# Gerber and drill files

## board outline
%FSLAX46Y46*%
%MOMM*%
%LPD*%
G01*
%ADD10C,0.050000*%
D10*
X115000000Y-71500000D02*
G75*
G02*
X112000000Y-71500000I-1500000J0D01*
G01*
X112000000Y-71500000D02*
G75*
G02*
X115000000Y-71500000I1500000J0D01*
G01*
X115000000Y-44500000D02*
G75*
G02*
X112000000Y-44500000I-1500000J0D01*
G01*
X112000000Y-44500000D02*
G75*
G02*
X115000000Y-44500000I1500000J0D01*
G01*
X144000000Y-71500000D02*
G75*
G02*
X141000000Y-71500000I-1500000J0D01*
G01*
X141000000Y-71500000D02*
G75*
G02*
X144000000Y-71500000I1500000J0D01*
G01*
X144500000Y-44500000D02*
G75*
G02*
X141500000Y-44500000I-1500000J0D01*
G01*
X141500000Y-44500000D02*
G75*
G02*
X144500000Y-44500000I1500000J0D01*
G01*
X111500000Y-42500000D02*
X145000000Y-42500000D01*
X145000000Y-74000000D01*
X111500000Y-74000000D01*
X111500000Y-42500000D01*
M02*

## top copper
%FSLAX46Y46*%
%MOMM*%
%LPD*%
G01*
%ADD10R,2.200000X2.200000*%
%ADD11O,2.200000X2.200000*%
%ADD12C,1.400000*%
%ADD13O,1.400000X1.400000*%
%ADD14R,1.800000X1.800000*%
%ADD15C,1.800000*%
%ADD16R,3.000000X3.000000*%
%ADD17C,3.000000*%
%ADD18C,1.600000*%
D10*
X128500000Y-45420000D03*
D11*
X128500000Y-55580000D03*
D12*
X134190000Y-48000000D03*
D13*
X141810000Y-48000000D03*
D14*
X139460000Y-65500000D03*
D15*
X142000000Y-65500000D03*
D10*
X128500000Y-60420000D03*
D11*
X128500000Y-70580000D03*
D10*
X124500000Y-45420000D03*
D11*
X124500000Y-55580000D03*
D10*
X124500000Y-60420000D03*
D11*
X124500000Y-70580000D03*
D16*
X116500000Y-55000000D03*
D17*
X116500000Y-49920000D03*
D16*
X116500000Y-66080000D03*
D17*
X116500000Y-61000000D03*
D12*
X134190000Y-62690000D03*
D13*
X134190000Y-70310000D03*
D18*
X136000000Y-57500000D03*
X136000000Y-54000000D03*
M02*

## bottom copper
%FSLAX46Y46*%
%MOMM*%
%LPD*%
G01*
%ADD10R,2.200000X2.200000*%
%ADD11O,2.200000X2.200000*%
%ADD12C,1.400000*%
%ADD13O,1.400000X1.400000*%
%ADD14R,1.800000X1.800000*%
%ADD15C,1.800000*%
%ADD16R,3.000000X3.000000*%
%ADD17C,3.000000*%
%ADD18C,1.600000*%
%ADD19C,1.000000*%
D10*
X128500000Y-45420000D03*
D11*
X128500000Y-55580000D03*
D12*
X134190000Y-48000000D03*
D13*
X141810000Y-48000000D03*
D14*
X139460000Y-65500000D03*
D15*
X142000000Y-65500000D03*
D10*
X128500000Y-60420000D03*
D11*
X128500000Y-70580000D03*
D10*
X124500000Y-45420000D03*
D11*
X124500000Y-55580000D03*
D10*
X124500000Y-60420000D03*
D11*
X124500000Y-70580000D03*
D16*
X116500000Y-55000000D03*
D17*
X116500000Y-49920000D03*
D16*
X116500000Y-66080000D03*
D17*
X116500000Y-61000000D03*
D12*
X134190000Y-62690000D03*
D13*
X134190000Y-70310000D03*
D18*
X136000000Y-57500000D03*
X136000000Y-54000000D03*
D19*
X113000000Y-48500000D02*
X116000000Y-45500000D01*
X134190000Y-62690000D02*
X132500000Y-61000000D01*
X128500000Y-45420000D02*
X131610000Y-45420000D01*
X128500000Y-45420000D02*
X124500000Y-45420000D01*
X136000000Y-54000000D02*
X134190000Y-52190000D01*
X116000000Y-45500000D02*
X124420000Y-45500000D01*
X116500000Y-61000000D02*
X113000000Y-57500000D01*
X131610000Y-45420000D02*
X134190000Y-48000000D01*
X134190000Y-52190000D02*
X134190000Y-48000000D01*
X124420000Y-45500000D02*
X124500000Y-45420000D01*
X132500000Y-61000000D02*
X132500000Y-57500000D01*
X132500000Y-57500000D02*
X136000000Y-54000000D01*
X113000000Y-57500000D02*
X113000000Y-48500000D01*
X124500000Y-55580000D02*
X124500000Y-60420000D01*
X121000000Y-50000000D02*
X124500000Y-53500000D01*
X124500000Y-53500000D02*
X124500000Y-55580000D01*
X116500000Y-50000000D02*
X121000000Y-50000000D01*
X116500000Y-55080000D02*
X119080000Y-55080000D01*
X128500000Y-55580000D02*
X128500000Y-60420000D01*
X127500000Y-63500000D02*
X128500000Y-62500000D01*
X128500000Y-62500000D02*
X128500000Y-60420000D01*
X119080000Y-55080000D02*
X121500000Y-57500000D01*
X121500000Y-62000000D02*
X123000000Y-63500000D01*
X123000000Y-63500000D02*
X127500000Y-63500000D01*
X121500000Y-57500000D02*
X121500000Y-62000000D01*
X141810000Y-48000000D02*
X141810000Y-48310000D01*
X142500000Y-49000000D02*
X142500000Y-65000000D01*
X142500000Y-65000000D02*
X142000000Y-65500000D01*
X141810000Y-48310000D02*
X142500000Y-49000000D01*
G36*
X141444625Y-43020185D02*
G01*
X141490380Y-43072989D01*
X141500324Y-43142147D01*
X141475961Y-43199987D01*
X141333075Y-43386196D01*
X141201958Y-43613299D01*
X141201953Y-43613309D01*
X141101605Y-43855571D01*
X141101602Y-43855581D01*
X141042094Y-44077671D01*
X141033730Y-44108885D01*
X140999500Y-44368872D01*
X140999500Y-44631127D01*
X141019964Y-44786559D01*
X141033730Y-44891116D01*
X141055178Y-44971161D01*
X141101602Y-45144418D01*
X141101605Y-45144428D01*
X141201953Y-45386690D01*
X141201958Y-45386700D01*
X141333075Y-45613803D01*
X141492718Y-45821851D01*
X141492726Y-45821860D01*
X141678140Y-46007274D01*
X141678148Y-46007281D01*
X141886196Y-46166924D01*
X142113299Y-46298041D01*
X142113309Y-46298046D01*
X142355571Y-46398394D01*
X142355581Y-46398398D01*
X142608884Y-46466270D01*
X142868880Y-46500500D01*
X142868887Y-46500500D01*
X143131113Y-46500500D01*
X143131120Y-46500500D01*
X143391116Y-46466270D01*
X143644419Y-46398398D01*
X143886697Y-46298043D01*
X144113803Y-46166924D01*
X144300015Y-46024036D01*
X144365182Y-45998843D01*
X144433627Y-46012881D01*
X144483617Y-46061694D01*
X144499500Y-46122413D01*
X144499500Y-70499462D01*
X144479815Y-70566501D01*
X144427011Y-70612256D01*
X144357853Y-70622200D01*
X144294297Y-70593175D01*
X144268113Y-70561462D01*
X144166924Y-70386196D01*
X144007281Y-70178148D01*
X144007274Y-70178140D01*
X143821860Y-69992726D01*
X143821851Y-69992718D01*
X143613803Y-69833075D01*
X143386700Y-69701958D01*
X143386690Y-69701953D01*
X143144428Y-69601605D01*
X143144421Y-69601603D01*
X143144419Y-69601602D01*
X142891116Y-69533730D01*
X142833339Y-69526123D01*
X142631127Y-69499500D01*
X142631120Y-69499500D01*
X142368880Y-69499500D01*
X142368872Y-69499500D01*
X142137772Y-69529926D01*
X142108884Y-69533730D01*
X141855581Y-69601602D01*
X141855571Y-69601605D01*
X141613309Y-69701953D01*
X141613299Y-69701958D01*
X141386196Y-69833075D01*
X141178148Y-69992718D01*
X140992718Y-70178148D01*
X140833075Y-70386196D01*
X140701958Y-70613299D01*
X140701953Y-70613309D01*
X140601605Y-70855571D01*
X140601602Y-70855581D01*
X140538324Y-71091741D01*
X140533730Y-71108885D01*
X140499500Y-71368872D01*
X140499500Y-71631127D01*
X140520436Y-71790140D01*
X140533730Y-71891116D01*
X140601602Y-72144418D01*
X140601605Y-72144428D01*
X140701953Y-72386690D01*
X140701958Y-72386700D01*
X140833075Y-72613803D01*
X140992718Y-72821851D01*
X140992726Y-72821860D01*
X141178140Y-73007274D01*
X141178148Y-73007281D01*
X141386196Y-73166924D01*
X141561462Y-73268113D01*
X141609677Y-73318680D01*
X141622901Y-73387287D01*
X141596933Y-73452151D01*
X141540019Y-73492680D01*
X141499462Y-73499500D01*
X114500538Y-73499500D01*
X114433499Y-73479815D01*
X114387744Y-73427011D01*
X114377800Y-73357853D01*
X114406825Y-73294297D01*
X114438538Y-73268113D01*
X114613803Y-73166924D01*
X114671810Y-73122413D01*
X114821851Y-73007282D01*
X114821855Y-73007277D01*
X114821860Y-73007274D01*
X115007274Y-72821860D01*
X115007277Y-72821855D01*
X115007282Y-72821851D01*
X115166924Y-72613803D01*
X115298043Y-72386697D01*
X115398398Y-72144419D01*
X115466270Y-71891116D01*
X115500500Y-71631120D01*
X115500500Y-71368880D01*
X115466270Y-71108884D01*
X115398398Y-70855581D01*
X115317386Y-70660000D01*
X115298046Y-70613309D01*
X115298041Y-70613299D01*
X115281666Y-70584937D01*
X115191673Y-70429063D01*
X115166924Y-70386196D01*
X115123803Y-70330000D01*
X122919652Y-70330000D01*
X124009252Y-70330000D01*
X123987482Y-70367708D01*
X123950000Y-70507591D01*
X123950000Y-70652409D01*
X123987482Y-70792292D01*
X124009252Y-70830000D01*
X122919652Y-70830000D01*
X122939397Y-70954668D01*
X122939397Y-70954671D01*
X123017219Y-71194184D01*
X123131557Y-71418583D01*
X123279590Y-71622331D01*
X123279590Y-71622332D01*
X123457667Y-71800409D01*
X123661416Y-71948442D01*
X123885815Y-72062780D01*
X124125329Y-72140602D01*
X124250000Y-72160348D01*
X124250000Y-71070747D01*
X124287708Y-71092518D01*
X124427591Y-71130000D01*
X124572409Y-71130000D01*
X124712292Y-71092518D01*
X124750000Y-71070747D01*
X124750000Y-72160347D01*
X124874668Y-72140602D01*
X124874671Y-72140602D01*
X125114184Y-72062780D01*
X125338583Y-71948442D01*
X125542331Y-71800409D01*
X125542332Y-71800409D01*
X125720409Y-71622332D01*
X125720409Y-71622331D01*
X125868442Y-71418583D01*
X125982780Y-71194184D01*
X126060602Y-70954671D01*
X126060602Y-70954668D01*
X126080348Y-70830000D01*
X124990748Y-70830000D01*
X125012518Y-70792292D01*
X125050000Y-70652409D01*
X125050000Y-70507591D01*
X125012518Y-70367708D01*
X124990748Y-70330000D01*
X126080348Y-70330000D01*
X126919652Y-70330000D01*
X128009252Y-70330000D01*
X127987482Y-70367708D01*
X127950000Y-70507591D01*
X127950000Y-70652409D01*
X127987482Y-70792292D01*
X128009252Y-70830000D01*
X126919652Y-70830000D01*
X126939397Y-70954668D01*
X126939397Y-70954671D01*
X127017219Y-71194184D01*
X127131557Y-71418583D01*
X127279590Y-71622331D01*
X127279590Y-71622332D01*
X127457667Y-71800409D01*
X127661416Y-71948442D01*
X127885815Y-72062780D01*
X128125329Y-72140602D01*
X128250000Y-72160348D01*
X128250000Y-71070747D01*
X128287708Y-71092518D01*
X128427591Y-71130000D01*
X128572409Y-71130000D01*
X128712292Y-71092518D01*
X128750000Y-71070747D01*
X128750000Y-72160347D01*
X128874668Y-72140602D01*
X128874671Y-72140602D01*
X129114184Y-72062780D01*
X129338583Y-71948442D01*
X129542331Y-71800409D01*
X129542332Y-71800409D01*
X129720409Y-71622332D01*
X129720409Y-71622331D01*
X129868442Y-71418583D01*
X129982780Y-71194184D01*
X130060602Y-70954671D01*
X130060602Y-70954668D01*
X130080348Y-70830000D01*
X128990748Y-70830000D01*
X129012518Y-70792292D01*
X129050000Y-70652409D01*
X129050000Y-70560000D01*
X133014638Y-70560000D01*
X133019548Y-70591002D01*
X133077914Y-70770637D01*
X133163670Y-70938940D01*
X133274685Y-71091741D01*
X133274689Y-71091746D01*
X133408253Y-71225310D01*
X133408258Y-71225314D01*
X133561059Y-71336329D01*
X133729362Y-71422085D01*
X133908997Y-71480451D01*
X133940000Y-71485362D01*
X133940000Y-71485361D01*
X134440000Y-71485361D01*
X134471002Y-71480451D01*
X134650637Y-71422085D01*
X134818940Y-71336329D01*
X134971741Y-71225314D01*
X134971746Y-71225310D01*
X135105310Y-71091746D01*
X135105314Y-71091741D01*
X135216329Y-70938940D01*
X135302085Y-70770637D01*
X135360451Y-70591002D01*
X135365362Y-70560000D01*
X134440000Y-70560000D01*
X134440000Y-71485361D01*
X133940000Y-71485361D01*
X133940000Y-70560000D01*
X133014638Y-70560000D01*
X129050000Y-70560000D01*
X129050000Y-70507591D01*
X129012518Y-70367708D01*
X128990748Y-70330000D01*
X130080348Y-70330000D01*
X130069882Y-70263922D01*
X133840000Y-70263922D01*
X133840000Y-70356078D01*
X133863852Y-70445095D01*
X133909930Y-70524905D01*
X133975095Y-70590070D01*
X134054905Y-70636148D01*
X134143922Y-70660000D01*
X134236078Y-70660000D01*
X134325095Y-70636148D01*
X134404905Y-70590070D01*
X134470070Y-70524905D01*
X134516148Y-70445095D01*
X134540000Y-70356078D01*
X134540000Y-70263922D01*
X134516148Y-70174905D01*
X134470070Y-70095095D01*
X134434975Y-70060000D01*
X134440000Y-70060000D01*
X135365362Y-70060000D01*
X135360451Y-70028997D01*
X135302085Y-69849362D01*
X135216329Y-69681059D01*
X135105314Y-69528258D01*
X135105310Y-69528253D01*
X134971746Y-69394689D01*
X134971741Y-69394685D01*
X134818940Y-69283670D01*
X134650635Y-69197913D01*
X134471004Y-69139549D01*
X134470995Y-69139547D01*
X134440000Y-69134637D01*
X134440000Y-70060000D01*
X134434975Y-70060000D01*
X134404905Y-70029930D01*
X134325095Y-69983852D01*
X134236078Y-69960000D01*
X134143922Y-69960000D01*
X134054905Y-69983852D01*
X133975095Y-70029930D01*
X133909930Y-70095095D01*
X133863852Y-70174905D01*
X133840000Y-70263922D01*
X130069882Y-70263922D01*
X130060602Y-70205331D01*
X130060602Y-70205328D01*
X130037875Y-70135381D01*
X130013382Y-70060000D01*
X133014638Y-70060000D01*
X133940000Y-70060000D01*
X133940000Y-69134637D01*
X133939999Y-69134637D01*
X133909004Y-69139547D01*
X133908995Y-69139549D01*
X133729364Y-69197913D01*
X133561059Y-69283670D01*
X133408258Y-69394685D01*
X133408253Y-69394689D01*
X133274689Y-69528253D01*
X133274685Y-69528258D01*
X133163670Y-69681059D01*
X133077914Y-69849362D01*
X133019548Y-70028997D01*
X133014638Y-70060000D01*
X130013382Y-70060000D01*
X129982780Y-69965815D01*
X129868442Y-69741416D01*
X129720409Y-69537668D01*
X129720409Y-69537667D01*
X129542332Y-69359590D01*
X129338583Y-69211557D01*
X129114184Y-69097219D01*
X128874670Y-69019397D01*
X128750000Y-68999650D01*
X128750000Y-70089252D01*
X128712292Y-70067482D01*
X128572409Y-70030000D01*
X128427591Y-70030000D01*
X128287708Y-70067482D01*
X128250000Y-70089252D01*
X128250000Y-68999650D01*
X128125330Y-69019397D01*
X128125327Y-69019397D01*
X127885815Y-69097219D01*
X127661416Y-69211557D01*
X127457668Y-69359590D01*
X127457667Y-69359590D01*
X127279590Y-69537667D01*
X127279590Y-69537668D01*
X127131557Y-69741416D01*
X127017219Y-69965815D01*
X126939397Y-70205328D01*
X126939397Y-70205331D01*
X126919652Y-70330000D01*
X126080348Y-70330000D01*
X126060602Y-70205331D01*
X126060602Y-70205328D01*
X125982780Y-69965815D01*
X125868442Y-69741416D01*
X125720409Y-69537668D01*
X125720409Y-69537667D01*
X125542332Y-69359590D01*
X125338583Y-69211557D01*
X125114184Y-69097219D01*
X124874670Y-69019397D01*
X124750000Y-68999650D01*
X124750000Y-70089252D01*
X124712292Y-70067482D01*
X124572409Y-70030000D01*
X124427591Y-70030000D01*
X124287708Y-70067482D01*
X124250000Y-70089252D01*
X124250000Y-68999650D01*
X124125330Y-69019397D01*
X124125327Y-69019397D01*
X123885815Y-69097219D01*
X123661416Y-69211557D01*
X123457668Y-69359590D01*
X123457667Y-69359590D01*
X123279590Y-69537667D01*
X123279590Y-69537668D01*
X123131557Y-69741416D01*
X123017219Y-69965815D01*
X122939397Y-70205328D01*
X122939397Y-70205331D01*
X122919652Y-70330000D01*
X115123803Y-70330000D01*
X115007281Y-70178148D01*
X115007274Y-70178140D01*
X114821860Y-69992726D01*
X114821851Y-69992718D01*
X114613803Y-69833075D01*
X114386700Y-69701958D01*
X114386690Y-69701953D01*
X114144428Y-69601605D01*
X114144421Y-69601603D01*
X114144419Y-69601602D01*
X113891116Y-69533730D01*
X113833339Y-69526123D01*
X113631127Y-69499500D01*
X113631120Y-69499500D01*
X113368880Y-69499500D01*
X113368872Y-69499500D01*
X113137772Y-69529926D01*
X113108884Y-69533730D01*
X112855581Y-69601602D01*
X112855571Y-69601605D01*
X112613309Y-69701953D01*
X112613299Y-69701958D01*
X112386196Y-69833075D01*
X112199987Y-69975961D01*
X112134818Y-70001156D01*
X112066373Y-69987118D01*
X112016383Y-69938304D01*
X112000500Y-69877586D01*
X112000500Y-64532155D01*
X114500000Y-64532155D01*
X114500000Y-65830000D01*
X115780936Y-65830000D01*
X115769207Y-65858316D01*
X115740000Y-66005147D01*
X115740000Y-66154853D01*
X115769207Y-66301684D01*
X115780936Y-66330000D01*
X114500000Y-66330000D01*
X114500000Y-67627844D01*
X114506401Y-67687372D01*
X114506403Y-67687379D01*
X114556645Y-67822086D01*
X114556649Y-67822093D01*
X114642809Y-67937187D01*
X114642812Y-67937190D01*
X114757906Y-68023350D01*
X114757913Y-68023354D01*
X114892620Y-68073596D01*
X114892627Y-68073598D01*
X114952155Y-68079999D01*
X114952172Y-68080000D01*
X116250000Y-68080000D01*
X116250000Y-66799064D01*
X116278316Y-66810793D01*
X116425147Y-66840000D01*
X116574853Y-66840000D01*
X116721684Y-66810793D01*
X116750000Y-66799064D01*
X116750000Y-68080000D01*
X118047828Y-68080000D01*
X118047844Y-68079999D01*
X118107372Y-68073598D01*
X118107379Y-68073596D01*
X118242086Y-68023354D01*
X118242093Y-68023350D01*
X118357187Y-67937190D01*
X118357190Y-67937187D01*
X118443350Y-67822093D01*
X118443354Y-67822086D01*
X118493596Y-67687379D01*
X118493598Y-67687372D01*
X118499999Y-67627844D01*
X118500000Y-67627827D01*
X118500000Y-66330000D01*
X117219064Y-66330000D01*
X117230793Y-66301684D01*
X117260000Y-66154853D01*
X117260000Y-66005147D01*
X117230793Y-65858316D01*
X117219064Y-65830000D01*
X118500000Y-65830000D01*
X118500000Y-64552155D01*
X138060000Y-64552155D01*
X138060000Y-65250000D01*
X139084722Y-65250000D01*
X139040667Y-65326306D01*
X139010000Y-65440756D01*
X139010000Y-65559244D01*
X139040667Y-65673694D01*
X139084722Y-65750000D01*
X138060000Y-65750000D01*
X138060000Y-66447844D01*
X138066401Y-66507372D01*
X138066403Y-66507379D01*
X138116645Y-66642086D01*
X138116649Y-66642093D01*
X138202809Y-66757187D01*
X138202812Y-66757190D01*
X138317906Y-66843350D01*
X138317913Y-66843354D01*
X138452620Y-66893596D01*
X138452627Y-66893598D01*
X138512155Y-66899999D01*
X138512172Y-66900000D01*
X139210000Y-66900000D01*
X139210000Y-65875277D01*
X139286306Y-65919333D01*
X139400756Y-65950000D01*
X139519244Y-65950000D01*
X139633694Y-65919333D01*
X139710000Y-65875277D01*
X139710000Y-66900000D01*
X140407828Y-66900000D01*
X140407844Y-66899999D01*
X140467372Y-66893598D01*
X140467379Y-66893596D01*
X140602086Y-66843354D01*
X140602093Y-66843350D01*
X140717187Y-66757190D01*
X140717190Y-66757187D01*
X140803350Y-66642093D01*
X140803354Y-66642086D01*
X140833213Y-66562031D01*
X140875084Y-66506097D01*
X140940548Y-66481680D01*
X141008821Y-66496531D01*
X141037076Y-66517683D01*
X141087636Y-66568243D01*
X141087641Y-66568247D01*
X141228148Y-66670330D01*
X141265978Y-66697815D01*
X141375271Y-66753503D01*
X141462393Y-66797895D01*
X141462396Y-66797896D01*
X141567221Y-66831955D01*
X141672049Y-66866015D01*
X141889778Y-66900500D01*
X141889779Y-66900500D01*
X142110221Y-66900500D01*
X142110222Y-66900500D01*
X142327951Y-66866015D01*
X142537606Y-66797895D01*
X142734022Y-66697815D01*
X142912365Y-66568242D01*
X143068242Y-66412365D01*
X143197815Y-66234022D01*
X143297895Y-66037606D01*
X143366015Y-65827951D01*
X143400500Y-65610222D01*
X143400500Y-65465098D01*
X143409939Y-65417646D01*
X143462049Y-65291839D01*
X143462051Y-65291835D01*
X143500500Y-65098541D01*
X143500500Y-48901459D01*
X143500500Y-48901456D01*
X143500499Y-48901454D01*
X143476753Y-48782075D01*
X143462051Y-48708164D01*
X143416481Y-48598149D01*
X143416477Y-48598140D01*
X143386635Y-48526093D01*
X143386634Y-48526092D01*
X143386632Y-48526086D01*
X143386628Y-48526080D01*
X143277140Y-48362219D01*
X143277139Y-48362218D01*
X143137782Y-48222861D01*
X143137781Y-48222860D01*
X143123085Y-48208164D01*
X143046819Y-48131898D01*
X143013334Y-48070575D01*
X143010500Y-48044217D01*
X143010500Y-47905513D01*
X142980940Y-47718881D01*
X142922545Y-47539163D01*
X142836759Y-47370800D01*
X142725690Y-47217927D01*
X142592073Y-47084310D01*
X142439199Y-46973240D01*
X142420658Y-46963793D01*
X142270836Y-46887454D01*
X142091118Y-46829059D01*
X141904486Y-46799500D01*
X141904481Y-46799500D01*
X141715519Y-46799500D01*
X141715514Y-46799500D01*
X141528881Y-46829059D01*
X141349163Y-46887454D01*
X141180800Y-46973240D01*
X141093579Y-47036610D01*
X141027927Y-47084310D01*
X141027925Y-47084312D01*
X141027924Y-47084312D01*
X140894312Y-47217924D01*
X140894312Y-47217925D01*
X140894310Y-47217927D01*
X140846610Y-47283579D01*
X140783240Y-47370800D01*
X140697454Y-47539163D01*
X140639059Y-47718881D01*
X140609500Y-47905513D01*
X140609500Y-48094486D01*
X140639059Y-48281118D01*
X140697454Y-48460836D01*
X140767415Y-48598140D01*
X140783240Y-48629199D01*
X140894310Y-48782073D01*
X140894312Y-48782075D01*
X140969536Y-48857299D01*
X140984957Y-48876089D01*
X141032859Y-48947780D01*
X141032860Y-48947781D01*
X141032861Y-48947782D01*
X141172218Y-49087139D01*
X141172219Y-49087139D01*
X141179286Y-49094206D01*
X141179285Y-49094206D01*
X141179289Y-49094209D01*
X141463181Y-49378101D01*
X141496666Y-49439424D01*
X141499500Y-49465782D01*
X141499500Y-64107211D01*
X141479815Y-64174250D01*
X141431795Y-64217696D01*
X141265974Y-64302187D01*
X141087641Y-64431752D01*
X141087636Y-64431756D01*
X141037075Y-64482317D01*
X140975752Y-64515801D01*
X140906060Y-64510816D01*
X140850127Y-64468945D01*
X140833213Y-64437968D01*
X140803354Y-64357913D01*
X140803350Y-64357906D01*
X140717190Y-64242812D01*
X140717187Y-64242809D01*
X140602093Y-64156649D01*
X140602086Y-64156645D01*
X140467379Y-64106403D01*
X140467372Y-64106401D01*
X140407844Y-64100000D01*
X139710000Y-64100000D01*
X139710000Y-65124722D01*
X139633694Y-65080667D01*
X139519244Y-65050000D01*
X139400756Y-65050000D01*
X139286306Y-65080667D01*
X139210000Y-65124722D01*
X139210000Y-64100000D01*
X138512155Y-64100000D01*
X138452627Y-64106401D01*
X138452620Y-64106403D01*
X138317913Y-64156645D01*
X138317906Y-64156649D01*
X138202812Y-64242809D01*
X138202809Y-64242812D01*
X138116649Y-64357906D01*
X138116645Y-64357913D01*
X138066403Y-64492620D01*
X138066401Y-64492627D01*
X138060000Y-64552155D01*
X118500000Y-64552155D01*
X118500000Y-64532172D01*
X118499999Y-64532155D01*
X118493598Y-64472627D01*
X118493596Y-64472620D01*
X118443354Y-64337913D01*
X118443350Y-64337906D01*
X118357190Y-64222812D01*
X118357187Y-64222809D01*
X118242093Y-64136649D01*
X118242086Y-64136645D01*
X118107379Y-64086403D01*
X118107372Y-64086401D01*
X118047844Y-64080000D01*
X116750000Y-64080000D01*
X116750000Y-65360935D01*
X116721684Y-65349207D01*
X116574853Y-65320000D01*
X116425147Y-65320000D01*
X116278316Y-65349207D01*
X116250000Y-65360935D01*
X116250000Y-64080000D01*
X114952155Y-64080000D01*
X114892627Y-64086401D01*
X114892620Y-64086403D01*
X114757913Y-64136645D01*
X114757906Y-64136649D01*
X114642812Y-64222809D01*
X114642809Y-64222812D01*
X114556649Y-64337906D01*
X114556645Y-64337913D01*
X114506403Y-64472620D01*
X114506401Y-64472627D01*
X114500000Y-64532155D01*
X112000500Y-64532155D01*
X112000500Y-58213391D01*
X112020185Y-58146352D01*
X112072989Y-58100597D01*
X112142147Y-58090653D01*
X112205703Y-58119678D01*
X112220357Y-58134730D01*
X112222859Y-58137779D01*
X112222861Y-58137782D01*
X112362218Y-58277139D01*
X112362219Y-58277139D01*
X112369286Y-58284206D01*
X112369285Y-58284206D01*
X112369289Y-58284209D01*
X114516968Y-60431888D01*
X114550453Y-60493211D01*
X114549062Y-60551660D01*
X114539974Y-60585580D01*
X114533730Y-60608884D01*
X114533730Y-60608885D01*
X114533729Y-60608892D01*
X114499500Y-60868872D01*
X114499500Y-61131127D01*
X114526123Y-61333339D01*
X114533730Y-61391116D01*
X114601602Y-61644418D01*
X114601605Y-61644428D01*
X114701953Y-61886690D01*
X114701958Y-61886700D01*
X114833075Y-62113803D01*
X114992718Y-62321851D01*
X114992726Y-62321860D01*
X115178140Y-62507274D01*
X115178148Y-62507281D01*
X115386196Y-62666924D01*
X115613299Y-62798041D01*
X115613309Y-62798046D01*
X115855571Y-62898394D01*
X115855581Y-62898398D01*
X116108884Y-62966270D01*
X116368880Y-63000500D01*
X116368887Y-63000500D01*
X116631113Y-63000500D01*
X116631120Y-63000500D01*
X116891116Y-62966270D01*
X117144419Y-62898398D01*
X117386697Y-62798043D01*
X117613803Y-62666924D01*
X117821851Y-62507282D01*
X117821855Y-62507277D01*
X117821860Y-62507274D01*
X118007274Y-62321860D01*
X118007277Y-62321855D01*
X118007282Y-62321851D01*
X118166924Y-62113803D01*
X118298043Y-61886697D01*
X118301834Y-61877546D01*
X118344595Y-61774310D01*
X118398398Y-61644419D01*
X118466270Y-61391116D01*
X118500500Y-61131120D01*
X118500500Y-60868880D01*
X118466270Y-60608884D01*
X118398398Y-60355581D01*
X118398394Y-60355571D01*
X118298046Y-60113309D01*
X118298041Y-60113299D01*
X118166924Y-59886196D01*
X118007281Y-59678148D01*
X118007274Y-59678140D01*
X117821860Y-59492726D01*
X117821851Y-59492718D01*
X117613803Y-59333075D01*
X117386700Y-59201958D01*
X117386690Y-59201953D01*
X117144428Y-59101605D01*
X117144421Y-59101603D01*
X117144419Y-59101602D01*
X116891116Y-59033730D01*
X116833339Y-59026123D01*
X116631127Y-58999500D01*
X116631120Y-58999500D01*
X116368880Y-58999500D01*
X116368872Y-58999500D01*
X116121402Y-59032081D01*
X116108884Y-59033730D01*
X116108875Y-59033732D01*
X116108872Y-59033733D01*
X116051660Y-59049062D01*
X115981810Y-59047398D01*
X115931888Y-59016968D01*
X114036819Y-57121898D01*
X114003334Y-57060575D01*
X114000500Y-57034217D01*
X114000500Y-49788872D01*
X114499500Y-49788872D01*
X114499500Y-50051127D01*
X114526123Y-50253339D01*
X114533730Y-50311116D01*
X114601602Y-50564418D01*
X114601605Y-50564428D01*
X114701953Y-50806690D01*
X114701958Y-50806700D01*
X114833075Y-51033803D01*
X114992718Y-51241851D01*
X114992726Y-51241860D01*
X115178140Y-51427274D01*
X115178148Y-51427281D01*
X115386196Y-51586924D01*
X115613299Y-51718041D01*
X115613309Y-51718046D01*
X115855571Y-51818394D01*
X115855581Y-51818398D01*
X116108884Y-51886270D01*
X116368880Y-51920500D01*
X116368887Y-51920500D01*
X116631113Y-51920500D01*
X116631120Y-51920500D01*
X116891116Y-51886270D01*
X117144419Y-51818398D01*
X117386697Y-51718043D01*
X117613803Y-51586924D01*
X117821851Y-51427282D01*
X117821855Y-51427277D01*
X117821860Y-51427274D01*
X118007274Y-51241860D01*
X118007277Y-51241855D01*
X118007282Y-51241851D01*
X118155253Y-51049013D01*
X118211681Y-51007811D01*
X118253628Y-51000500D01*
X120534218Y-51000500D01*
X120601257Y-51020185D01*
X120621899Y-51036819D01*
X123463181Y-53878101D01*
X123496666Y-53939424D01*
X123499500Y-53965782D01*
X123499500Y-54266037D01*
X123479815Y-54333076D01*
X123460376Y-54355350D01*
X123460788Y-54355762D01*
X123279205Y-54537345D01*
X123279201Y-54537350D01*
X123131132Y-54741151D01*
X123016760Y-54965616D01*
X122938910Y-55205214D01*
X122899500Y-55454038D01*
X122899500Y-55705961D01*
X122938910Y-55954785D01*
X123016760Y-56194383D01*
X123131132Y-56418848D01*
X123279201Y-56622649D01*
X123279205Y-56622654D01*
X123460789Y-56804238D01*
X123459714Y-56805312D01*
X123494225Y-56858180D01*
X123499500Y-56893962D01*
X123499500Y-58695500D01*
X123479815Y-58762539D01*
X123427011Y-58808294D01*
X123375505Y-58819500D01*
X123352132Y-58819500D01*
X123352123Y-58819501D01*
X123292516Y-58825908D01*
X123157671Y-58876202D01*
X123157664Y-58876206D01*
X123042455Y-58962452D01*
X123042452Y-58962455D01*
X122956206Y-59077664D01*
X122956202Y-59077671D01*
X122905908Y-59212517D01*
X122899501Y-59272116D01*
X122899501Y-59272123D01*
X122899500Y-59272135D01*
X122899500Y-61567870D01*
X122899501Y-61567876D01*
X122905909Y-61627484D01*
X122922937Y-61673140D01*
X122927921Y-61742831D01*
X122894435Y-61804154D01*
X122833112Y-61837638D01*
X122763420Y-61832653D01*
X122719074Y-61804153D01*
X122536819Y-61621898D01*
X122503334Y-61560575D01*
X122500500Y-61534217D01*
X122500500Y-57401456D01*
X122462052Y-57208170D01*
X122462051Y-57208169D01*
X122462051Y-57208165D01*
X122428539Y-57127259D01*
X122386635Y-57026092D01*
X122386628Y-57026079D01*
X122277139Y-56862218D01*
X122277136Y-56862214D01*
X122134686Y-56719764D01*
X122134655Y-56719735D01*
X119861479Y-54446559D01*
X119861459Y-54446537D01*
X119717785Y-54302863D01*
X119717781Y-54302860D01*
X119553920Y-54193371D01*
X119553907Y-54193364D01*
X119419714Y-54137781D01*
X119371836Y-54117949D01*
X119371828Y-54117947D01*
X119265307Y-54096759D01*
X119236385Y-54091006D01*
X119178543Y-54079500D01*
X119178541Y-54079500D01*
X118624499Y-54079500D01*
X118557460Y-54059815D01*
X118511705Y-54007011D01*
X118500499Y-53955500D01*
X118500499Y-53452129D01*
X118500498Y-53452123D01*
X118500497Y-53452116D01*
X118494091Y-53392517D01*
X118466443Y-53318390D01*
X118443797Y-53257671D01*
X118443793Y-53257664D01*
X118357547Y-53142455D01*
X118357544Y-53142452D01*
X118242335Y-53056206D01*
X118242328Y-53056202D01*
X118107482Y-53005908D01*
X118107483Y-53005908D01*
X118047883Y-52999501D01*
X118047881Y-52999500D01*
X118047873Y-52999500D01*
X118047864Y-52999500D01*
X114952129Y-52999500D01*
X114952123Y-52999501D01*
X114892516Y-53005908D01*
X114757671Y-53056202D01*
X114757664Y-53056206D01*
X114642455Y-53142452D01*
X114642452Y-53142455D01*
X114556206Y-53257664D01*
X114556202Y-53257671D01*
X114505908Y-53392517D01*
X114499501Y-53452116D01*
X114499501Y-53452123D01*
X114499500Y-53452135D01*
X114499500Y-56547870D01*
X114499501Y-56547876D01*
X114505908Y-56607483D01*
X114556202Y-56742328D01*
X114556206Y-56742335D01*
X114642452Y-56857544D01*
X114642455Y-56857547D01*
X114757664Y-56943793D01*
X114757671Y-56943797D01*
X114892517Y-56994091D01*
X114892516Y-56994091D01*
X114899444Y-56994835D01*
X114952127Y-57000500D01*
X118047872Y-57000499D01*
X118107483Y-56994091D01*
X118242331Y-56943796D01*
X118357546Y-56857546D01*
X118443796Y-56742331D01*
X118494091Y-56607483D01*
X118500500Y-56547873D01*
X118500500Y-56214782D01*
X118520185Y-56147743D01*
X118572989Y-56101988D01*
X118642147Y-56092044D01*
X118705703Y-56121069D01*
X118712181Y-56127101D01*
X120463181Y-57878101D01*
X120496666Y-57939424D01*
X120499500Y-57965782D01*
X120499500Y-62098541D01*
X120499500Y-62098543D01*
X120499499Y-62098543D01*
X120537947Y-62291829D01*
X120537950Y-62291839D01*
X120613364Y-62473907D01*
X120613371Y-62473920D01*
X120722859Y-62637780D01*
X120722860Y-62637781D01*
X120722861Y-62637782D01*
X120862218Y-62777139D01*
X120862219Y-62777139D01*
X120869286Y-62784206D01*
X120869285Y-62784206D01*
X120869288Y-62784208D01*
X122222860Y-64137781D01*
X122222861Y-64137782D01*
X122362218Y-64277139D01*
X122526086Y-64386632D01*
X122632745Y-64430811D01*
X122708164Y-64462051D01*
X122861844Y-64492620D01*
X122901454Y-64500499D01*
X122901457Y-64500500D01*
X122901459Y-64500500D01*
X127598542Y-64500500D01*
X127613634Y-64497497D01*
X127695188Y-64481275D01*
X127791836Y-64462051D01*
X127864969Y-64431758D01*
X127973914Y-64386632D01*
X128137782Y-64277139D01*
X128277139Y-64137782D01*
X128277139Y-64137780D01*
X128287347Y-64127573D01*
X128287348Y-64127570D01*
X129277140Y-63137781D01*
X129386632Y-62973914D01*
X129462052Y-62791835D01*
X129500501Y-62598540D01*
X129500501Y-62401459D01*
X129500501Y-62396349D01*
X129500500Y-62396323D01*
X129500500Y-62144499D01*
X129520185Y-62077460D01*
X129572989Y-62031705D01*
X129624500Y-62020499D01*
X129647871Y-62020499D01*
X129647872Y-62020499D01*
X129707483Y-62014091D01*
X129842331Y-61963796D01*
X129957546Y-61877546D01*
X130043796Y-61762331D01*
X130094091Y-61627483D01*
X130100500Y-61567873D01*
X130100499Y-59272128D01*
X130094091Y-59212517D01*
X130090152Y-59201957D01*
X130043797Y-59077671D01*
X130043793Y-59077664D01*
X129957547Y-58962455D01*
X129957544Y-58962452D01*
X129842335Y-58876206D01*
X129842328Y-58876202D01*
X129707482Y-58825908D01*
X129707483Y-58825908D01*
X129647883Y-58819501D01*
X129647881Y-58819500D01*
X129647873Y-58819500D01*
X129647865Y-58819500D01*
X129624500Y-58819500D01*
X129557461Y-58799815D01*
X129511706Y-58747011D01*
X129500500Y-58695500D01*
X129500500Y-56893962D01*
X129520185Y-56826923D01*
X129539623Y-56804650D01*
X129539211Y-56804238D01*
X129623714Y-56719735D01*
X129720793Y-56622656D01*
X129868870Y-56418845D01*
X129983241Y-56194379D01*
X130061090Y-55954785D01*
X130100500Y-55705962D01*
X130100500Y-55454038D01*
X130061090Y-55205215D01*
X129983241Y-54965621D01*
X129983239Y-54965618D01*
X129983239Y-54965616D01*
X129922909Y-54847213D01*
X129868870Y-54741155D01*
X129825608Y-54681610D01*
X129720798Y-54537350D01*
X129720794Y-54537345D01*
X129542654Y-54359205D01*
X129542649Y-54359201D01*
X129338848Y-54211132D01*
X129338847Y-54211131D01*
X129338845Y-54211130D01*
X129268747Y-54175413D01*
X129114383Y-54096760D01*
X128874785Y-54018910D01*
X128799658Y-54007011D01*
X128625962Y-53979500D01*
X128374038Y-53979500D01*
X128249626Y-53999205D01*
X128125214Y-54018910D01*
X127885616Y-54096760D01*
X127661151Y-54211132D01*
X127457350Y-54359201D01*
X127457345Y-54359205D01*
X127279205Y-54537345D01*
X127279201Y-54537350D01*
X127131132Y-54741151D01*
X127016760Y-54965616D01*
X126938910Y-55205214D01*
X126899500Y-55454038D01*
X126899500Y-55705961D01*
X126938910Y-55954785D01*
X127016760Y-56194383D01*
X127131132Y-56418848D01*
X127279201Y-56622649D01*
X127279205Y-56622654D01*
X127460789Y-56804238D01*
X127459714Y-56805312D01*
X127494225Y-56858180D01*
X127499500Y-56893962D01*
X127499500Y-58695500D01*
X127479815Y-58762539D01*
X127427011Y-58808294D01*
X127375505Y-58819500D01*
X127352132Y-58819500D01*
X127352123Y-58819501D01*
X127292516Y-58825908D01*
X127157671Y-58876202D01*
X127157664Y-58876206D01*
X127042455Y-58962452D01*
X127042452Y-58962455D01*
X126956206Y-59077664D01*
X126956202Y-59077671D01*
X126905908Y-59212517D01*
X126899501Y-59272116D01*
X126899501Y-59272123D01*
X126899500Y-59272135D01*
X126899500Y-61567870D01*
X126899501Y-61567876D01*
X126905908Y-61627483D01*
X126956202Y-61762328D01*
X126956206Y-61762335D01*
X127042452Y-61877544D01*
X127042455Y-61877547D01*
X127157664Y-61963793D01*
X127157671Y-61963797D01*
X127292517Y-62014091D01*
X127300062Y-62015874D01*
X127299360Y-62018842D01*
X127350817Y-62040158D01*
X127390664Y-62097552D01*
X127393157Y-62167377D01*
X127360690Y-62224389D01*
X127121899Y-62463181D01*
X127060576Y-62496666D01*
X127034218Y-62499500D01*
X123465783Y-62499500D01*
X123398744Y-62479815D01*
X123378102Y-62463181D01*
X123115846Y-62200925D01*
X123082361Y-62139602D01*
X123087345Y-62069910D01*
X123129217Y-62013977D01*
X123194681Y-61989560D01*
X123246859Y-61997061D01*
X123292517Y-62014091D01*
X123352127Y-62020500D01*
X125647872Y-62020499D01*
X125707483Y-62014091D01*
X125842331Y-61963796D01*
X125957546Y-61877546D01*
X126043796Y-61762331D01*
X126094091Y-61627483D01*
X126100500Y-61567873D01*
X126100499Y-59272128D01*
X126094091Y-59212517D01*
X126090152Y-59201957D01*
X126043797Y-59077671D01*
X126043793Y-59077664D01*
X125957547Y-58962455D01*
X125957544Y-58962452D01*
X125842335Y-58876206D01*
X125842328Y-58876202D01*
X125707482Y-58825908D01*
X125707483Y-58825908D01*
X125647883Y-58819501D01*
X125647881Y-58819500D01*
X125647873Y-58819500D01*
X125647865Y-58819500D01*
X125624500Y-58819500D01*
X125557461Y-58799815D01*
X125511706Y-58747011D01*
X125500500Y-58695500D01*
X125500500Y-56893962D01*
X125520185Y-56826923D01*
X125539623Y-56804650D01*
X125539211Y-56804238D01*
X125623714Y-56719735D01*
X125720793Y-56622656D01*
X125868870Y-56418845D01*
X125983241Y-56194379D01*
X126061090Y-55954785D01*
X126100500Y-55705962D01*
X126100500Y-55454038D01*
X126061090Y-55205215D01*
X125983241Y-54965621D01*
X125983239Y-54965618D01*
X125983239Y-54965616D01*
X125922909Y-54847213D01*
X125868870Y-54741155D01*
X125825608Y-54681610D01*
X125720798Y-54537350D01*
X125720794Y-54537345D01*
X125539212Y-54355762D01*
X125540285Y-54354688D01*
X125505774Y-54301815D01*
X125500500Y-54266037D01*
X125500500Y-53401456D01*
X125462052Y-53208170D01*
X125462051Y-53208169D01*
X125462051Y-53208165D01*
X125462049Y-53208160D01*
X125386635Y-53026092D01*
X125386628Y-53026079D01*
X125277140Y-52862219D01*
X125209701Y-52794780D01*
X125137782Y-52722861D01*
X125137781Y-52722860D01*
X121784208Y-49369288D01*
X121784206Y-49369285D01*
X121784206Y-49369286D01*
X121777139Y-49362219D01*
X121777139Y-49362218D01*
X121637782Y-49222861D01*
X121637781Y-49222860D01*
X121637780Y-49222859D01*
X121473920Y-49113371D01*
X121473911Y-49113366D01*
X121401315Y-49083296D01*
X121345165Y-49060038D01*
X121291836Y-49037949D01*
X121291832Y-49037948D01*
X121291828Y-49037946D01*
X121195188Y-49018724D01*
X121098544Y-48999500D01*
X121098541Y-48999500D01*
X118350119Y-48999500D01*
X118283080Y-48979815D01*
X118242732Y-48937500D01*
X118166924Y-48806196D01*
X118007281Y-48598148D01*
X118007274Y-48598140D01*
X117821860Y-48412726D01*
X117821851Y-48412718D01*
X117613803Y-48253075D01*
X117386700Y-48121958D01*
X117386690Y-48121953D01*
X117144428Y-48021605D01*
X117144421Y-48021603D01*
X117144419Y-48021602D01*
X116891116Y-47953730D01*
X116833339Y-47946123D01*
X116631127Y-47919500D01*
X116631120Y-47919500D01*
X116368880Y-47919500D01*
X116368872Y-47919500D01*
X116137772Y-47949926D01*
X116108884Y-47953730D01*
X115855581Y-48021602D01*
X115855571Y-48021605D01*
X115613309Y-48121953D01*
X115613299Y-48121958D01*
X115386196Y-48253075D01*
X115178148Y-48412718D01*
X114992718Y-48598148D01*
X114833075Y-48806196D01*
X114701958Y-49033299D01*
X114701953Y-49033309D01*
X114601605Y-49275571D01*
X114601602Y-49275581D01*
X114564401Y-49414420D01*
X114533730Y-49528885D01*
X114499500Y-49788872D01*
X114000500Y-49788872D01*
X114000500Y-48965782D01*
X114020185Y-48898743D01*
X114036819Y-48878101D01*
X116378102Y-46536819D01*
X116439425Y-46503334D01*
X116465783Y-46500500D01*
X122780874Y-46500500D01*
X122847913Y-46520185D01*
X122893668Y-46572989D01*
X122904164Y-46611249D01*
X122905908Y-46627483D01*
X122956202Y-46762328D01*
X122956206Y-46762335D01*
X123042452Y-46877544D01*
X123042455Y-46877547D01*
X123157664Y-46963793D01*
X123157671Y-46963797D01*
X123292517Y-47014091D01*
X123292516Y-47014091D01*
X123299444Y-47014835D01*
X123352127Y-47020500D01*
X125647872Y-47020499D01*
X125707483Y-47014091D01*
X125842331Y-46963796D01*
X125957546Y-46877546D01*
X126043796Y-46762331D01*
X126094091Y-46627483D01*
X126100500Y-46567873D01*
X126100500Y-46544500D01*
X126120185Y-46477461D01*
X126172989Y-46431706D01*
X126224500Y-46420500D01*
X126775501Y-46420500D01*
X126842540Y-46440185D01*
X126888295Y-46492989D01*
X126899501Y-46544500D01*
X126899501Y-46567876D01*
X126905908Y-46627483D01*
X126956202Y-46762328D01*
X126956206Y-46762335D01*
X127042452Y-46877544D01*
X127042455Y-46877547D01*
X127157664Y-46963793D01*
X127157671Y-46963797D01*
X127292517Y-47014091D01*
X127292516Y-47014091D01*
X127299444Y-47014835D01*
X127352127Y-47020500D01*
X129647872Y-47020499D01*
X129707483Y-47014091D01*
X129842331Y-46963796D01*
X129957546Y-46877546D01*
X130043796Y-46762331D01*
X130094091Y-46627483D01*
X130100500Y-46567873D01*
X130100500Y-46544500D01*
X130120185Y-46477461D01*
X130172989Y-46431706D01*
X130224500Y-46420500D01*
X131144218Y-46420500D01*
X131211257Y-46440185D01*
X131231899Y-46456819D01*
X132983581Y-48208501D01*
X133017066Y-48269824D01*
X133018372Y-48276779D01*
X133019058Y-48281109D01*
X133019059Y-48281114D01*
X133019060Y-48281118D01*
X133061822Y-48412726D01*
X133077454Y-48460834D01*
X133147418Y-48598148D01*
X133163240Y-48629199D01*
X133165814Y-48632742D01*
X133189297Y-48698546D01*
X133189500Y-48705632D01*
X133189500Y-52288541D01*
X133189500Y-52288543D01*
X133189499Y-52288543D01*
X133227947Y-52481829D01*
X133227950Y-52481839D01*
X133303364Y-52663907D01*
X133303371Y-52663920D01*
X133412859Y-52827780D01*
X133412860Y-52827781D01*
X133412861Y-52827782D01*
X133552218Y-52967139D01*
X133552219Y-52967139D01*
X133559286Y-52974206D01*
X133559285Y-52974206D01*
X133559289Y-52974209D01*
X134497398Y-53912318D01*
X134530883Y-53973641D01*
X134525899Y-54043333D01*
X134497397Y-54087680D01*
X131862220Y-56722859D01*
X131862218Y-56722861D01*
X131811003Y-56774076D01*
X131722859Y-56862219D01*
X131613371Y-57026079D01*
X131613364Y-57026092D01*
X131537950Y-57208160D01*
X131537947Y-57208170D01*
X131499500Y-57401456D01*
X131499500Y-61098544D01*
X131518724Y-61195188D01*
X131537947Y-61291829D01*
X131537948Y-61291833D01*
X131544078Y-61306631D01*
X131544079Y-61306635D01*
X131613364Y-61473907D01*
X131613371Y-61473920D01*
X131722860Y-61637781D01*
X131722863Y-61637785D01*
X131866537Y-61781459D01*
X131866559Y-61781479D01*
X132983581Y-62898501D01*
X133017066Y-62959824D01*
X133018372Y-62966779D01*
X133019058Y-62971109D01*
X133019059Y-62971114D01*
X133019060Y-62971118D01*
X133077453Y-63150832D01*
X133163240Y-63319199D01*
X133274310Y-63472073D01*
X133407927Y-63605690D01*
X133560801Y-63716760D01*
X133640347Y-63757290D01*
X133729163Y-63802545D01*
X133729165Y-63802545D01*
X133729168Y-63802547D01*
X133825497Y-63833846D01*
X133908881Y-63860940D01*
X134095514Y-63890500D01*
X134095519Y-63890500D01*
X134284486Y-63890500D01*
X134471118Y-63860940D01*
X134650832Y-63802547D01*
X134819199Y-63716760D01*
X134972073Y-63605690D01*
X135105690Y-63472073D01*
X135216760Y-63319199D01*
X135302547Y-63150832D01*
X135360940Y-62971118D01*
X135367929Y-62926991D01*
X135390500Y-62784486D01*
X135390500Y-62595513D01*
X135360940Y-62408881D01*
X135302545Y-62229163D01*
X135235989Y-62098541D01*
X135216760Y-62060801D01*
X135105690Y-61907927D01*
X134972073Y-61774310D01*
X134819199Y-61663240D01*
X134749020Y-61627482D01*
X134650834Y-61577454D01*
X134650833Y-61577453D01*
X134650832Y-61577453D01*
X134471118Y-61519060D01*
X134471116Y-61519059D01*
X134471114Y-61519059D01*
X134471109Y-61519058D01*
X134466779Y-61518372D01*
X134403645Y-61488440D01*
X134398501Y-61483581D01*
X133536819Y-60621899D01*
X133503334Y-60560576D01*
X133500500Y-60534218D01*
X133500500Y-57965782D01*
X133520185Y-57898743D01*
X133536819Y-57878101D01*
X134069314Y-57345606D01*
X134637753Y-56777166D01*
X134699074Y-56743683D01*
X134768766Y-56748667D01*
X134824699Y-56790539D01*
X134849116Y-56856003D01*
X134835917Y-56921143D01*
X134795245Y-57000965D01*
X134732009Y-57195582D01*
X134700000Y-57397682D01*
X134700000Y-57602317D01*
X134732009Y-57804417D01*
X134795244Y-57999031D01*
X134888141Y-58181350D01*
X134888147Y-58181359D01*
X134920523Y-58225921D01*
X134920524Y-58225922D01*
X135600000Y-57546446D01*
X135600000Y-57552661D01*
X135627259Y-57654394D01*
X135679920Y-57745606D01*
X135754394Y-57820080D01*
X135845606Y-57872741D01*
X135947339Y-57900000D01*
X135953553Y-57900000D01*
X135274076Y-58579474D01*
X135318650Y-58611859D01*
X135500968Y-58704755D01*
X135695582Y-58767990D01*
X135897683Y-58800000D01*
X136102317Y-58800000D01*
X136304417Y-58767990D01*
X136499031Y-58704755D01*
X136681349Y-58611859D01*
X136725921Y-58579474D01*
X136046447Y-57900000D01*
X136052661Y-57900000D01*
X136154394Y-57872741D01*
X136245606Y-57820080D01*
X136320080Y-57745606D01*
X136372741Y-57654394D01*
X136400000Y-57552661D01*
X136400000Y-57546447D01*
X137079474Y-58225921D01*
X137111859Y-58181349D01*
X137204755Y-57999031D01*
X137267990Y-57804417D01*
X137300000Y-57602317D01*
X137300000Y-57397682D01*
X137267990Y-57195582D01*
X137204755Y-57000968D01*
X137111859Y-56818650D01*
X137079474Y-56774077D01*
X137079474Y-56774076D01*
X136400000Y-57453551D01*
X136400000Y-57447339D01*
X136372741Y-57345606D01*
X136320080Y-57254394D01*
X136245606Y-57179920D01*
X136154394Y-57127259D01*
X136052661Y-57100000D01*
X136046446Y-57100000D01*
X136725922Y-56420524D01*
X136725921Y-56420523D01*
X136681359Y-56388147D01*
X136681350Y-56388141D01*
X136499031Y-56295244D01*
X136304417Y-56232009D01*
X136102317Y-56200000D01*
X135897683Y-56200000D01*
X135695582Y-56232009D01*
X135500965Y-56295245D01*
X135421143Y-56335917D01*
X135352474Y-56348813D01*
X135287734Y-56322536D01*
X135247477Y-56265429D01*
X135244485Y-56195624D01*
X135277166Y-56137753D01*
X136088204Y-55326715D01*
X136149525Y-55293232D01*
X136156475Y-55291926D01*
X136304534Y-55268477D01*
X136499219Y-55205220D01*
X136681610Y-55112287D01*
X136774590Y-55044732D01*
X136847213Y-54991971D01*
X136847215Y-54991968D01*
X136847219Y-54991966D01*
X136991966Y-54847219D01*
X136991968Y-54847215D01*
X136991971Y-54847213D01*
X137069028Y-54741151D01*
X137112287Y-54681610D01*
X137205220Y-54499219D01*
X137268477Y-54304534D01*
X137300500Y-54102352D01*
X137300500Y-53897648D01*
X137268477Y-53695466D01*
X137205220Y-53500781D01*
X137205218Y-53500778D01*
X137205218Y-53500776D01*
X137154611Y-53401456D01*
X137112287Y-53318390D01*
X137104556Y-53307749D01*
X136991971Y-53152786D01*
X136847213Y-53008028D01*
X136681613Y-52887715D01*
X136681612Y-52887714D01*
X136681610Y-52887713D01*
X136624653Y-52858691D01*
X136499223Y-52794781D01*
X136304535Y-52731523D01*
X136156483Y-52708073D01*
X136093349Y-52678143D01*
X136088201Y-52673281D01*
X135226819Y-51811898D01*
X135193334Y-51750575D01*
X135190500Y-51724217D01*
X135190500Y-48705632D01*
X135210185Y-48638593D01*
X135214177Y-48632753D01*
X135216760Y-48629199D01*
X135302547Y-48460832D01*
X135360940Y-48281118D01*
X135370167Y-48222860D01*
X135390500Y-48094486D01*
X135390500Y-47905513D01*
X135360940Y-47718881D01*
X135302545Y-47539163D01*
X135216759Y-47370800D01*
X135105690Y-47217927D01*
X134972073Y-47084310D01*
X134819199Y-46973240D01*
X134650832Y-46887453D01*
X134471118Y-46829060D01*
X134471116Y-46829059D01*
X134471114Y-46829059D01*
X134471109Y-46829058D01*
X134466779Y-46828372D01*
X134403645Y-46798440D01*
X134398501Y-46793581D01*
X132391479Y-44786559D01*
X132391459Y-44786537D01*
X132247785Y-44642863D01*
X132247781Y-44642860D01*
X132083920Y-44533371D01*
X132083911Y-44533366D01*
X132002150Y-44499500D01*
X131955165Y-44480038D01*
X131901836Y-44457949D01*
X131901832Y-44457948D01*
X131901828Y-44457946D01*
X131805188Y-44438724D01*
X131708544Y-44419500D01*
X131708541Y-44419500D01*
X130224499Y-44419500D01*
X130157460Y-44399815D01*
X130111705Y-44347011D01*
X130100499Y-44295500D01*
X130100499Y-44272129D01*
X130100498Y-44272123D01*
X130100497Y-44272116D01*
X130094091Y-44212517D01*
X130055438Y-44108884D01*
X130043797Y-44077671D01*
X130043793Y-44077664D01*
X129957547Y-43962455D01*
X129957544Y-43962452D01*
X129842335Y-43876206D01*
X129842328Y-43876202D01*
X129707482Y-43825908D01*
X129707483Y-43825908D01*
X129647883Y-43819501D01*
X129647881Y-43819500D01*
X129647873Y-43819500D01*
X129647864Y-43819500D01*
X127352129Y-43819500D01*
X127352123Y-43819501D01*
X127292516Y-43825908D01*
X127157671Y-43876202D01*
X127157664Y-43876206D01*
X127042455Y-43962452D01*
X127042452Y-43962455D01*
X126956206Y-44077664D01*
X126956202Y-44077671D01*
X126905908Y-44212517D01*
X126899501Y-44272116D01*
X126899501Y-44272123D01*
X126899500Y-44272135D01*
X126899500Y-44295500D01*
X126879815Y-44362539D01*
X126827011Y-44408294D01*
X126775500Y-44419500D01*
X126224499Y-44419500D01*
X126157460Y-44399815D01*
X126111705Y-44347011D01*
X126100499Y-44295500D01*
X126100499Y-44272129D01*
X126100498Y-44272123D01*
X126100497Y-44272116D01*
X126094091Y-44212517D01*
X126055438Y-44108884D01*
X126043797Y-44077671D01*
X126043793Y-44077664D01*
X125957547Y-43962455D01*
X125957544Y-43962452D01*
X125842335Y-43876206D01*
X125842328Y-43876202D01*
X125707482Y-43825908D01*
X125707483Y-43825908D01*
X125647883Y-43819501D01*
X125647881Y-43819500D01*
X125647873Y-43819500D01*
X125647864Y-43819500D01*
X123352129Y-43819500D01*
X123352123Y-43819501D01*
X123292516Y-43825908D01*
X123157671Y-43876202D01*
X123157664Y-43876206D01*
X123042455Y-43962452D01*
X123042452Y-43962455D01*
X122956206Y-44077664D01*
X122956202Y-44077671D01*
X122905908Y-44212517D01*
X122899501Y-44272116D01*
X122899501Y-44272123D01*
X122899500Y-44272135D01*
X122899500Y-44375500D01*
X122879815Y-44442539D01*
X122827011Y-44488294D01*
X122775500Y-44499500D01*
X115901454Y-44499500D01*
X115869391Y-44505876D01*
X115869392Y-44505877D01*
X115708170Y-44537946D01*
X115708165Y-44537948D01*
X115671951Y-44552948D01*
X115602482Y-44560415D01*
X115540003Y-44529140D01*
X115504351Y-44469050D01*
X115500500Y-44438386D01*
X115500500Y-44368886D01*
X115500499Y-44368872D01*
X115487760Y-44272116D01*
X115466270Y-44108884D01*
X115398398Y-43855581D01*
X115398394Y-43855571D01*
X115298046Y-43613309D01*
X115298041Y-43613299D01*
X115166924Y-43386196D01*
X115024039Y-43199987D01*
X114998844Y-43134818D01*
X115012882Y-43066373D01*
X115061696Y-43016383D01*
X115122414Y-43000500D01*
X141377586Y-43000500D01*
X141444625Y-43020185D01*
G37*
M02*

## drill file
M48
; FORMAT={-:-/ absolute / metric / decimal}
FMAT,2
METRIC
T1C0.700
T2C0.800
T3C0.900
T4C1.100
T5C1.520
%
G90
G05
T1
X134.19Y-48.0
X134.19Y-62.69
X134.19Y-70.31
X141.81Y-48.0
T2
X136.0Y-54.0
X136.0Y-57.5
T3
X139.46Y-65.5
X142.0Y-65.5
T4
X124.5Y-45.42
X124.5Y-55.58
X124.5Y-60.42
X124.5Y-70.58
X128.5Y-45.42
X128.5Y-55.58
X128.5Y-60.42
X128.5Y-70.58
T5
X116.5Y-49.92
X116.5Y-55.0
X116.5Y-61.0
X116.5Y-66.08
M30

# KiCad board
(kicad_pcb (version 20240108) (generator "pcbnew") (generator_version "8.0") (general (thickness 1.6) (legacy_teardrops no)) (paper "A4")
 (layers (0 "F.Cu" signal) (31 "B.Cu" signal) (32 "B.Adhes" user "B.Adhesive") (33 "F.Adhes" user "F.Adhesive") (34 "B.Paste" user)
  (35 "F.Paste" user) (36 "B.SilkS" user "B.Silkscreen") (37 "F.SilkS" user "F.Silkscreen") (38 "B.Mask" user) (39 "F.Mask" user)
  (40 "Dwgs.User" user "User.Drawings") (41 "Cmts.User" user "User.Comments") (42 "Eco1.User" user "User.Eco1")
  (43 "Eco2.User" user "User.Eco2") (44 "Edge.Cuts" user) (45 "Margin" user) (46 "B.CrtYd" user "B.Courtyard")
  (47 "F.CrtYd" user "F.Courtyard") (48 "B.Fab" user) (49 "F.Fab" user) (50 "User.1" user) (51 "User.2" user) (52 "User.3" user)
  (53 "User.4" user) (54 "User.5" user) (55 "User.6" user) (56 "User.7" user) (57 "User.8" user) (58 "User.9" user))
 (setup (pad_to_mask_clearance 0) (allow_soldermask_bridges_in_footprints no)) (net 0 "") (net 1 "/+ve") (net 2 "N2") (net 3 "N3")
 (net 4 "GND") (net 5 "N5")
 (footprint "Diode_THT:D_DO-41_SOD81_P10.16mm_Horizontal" (layer "F.Cu") (at 128.5 45.42 -90)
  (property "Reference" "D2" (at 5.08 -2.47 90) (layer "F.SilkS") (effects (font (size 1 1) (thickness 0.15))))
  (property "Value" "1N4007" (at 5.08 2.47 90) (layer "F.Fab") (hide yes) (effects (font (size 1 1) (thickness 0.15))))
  (pad "1" thru_hole rect (at 0 0 270) (size 2.2 2.2) (drill 1.1) (layers "*.Cu" "*.Mask") (remove_unused_layers no) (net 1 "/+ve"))
  (pad "2" thru_hole oval (at 10.16 0 270) (size 2.2 2.2) (drill 1.1) (layers "*.Cu" "*.Mask") (remove_unused_layers no) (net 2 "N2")))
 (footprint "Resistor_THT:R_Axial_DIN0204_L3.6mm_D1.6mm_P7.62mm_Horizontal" (layer "F.Cu") (at 134.19 48)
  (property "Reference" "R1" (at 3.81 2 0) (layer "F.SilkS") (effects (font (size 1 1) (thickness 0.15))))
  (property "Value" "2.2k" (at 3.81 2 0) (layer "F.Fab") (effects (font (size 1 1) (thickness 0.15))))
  (pad "1" thru_hole circle (at 0 0) (size 1.4 1.4) (drill 0.7) (layers "*.Cu" "*.Mask") (remove_unused_layers no) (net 1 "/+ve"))
  (pad "2" thru_hole oval (at 7.62 0) (size 1.4 1.4) (drill 0.7) (layers "*.Cu" "*.Mask") (remove_unused_layers no) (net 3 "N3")))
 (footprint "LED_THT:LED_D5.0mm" (layer "F.Cu") (at 139.46 65.5)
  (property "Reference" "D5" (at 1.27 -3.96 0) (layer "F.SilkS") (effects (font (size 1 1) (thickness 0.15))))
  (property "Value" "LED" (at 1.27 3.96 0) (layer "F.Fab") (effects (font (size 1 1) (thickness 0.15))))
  (pad "1" thru_hole rect (at 0 0) (size 1.8 1.8) (drill 0.9) (layers "*.Cu" "*.Mask") (remove_unused_layers no) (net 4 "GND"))
  (pad "2" thru_hole circle (at 2.54 0) (size 1.8 1.8) (drill 0.9) (layers "*.Cu" "*.Mask") (remove_unused_layers no) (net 3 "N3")))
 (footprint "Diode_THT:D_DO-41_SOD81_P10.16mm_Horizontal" (layer "F.Cu") (at 128.5 60.42 -90)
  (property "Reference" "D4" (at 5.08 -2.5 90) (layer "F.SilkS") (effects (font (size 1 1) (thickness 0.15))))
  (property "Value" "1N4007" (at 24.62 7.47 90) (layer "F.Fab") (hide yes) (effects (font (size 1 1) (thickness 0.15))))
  (pad "1" thru_hole rect (at 0 0 270) (size 2.2 2.2) (drill 1.1) (layers "*.Cu" "*.Mask") (remove_unused_layers no) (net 2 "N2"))
  (pad "2" thru_hole oval (at 10.16 0 270) (size 2.2 2.2) (drill 1.1) (layers "*.Cu" "*.Mask") (remove_unused_layers no) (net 4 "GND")))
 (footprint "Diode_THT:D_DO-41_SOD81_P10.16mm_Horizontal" (layer "F.Cu") (at 124.5 45.42 -90)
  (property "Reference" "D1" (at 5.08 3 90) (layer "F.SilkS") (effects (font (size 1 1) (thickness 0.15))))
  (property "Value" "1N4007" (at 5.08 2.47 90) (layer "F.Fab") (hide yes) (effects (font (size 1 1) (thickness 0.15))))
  (pad "1" thru_hole rect (at 0 0 270) (size 2.2 2.2) (drill 1.1) (layers "*.Cu" "*.Mask") (remove_unused_layers no) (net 1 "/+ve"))
  (pad "2" thru_hole oval (at 10.16 0 270) (size 2.2 2.2) (drill 1.1) (layers "*.Cu" "*.Mask") (remove_unused_layers no) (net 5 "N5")))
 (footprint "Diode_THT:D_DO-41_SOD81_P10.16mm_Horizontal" (layer "F.Cu") (at 124.5 60.42 -90)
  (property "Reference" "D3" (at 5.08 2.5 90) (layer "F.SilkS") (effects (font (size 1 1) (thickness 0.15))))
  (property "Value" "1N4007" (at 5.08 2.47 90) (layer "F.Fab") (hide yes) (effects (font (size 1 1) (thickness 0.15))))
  (pad "1" thru_hole rect (at 0 0 270) (size 2.2 2.2) (drill 1.1) (layers "*.Cu" "*.Mask") (remove_unused_layers no) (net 5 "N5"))
  (pad "2" thru_hole oval (at 10.16 0 270) (size 2.2 2.2) (drill 1.1) (layers "*.Cu" "*.Mask") (remove_unused_layers no) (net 4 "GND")))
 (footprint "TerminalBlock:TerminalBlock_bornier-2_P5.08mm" (layer "F.Cu") (at 116.5 55 90)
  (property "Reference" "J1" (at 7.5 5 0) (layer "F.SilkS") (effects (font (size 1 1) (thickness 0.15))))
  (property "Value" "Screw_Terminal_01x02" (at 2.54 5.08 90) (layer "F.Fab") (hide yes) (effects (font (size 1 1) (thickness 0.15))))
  (pad "1" thru_hole rect (at 0 0 90) (size 3 3) (drill 1.52) (layers "*.Cu" "*.Mask") (remove_unused_layers no) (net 2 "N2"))
  (pad "2" thru_hole circle (at 5.08 0 90) (size 3 3) (drill 1.52) (layers "*.Cu" "*.Mask") (remove_unused_layers no) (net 5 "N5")))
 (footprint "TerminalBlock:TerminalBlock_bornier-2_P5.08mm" (layer "F.Cu") (at 116.5 66.08 90)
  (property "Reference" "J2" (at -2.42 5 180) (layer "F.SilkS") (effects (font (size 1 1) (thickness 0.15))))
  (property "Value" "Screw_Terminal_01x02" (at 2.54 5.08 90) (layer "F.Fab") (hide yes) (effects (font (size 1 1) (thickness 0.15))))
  (pad "1" thru_hole rect (at 0 0 90) (size 3 3) (drill 1.52) (layers "*.Cu" "*.Mask") (remove_unused_layers no) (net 4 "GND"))
  (pad "2" thru_hole circle (at 5.08 0 90) (size 3 3) (drill 1.52) (layers "*.Cu" "*.Mask") (remove_unused_layers no) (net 1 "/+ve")))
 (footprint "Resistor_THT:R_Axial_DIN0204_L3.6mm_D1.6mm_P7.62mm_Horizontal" (layer "F.Cu") (at 134.19 62.69 -90)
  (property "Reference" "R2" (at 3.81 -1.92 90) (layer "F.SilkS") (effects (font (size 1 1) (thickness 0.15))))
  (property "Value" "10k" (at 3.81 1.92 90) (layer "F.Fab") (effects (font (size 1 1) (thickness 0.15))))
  (pad "1" thru_hole circle (at 0 0 270) (size 1.4 1.4) (drill 0.7) (layers "*.Cu" "*.Mask") (remove_unused_layers no) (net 1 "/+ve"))
  (pad "2" thru_hole oval (at 7.62 0 270) (size 1.4 1.4) (drill 0.7) (layers "*.Cu" "*.Mask") (remove_unused_layers no) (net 4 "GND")))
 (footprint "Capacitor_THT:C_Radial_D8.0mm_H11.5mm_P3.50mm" (layer "F.Cu") (at 136 57.5 90)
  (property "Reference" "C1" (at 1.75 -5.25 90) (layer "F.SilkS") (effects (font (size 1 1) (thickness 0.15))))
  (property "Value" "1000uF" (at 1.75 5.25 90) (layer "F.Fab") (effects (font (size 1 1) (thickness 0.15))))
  (pad "1" thru_hole circle (at 0 0 90) (size 1.6 1.6) (drill 0.8) (layers "*.Cu" "*.Mask") (remove_unused_layers no) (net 4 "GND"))
  (pad "2" thru_hole circle (at 3.5 0 90) (size 1.6 1.6) (drill 0.8) (layers "*.Cu" "*.Mask") (remove_unused_layers no) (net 1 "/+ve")))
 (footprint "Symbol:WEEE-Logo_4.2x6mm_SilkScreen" (layer "B.Cu") (at 138.5 58.5 180)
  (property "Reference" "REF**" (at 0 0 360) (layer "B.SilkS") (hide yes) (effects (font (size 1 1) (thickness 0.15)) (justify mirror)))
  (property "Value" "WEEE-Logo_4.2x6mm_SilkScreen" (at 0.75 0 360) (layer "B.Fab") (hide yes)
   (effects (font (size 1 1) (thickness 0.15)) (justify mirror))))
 (gr_circle (center 113.5 71.5) (end 115 71.5) (stroke (width 0.05) (type default)) (fill none) (layer "Edge.Cuts"))
 (gr_circle (center 113.5 44.5) (end 115 44.5) (stroke (width 0.05) (type default)) (fill none) (layer "Edge.Cuts"))
 (gr_circle (center 142.5 71.5) (end 144 71.5) (stroke (width 0.05) (type default)) (fill none) (layer "Edge.Cuts"))
 (gr_circle (center 143 44.5) (end 144.5 44.5) (stroke (width 0.05) (type default)) (fill none) (layer "Edge.Cuts"))
 (gr_rect (start 111.5 42.5) (end 145 74) (stroke (width 0.05) (type default)) (fill none) (layer "Edge.Cuts"))
 (segment (start 113 48.5) (end 116 45.5) (width 1) (layer "B.Cu") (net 1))
 (segment (start 134.19 62.69) (end 132.5 61) (width 1) (layer "B.Cu") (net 1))
 (segment (start 128.5 45.42) (end 131.61 45.42) (width 1) (layer "B.Cu") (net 1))
 (segment (start 128.5 45.42) (end 124.5 45.42) (width 1) (layer "B.Cu") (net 1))
 (segment (start 136 54) (end 134.19 52.19) (width 1) (layer "B.Cu") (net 1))
 (segment (start 116 45.5) (end 124.42 45.5) (width 1) (layer "B.Cu") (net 1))
 (segment (start 116.5 61) (end 113 57.5) (width 1) (layer "B.Cu") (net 1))
 (segment (start 131.61 45.42) (end 134.19 48) (width 1) (layer "B.Cu") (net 1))
 (segment (start 134.19 52.19) (end 134.19 48) (width 1) (layer "B.Cu") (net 1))
 (segment (start 124.42 45.5) (end 124.5 45.42) (width 1) (layer "B.Cu") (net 1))
 (segment (start 132.5 61) (end 132.5 57.5) (width 1) (layer "B.Cu") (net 1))
 (segment (start 132.5 57.5) (end 136 54) (width 1) (layer "B.Cu") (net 1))
 (segment (start 113 57.5) (end 113 48.5) (width 1) (layer "B.Cu") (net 1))
 (segment (start 124.5 55.58) (end 124.5 60.42) (width 1) (layer "B.Cu") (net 5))
 (segment (start 121 50) (end 124.5 53.5) (width 1) (layer "B.Cu") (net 5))
 (segment (start 124.5 53.5) (end 124.5 55.58) (width 1) (layer "B.Cu") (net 5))
 (segment (start 116.5 50) (end 121 50) (width 1) (layer "B.Cu") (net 5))
 (segment (start 116.5 55.08) (end 119.08 55.08) (width 1) (layer "B.Cu") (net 2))
 (segment (start 128.5 55.58) (end 128.5 60.42) (width 1) (layer "B.Cu") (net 2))
 (segment (start 127.5 63.5) (end 128.5 62.5) (width 1) (layer "B.Cu") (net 2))
 (segment (start 128.5 62.5) (end 128.5 60.42) (width 1) (layer "B.Cu") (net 2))
 (segment (start 119.08 55.08) (end 121.5 57.5) (width 1) (layer "B.Cu") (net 2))
 (segment (start 121.5 62) (end 123 63.5) (width 1) (layer "B.Cu") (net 2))
 (segment (start 123 63.5) (end 127.5 63.5) (width 1) (layer "B.Cu") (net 2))
 (segment (start 121.5 57.5) (end 121.5 62) (width 1) (layer "B.Cu") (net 2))
 (segment (start 141.81 48) (end 141.81 48.31) (width 1) (layer "B.Cu") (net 3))
 (segment (start 142.5 49) (end 142.5 65) (width 1) (layer "B.Cu") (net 3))
 (segment (start 142.5 65) (end 142 65.5) (width 1) (layer "B.Cu") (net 3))
 (segment (start 141.81 48.31) (end 142.5 49) (width 1) (layer "B.Cu") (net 3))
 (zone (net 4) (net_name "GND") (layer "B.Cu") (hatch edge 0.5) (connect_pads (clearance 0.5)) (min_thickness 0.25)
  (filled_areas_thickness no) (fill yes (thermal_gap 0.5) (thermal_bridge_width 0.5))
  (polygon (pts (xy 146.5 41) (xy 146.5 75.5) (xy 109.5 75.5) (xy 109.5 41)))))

